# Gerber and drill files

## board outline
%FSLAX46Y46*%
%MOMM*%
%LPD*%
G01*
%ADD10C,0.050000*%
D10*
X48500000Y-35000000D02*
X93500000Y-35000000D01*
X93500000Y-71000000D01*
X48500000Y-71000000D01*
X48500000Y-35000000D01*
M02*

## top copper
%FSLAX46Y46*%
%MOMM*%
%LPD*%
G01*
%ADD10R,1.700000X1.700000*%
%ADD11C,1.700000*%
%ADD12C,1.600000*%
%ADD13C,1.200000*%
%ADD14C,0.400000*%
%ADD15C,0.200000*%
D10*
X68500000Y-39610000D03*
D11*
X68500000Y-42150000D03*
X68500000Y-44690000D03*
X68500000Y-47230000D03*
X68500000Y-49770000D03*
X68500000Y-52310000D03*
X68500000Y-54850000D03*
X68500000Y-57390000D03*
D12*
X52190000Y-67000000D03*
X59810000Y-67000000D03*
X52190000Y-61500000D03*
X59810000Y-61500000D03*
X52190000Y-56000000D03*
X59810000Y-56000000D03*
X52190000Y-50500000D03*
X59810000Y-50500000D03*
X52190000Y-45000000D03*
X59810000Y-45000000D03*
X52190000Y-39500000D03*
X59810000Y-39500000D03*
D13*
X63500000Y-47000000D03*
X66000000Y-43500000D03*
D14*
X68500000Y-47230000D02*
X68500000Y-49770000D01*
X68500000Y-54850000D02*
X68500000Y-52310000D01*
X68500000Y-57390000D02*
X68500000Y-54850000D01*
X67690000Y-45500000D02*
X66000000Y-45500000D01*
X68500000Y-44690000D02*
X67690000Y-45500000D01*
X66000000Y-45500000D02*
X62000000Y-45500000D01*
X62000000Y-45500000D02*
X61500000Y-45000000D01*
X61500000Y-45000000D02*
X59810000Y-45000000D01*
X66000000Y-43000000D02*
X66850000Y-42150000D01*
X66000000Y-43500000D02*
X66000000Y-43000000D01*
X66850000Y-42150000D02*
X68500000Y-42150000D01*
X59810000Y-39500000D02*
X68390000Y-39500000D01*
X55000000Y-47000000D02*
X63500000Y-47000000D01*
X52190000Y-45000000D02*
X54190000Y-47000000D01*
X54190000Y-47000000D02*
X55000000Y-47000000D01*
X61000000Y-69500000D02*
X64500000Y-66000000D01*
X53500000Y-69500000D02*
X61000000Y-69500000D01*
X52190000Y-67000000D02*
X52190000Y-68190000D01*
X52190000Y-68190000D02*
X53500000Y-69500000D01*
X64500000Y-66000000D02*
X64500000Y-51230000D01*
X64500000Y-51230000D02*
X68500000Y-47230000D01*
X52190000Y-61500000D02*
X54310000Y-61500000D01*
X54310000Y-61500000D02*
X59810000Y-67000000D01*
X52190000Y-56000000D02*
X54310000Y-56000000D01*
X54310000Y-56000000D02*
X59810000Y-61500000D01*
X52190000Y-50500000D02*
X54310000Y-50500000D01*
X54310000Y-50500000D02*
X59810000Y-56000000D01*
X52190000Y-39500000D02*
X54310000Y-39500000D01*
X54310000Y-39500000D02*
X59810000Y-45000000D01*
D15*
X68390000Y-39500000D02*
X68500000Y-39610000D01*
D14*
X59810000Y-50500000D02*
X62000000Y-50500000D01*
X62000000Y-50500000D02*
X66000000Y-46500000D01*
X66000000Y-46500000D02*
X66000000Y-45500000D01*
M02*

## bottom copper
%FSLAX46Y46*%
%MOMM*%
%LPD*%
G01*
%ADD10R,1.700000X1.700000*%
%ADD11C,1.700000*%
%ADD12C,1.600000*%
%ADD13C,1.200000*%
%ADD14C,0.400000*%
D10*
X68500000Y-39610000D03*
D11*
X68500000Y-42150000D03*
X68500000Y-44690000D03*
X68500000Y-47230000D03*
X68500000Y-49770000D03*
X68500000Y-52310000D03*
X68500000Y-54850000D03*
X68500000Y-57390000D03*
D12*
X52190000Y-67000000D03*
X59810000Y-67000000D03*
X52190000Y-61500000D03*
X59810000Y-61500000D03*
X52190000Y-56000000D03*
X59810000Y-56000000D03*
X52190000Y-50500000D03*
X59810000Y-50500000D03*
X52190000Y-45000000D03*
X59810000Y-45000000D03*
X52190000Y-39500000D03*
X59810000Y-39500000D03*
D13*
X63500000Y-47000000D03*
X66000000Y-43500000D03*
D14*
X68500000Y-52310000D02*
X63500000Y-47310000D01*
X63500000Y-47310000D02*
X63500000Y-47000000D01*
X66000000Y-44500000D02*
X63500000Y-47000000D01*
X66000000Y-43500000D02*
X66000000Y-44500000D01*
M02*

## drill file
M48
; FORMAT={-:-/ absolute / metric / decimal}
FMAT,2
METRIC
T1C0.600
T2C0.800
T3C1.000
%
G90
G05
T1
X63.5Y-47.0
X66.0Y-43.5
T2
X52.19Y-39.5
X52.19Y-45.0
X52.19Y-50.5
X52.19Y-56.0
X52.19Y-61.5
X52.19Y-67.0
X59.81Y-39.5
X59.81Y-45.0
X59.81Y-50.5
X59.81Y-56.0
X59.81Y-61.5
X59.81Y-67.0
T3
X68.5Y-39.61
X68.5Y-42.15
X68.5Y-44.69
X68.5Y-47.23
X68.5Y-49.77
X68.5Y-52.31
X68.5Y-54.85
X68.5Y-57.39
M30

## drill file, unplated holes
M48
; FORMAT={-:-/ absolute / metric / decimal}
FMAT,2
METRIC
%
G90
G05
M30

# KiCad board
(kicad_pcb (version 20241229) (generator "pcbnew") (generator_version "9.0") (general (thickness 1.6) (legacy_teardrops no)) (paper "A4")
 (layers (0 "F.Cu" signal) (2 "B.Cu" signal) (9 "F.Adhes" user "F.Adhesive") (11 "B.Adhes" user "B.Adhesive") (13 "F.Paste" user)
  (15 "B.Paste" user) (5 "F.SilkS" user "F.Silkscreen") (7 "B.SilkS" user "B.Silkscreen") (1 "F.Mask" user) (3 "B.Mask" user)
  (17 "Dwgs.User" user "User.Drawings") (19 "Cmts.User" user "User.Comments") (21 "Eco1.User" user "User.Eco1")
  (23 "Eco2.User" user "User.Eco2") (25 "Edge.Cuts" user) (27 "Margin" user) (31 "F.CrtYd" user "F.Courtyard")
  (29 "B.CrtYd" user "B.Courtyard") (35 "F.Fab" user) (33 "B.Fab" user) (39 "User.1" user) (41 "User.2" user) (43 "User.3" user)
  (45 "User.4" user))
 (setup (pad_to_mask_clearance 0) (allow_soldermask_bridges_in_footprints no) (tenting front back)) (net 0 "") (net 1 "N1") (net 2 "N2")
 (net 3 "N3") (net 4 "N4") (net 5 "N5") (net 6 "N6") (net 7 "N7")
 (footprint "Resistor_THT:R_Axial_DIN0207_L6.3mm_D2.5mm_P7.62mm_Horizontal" (layer "F.Cu") (at 52.19 45)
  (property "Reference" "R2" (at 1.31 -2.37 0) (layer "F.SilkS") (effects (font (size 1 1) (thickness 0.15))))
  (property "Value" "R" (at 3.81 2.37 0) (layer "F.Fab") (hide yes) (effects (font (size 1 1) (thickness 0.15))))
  (pad "1" thru_hole circle (at 0 0) (size 1.6 1.6) (drill 0.8) (layers "*.Cu" "*.Mask") (remove_unused_layers no) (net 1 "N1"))
  (pad "2" thru_hole circle (at 7.62 0) (size 1.6 1.6) (drill 0.8) (layers "*.Cu" "*.Mask") (remove_unused_layers no) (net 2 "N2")))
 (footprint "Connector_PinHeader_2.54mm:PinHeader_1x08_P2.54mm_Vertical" (layer "F.Cu") (at 68.5 39.61)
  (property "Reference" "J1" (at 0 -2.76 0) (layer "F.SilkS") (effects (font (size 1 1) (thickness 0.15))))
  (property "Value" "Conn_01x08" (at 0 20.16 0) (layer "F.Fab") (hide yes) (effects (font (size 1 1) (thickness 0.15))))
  (pad "1" thru_hole rect (at 0 0) (size 1.7 1.7) (drill 1) (layers "*.Cu" "*.Mask") (remove_unused_layers no) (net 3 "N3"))
  (pad "2" thru_hole circle (at 0 2.54) (size 1.7 1.7) (drill 1) (layers "*.Cu" "*.Mask") (remove_unused_layers no) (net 1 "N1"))
  (pad "3" thru_hole circle (at 0 5.08) (size 1.7 1.7) (drill 1) (layers "*.Cu" "*.Mask") (remove_unused_layers no) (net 2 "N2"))
  (pad "4" thru_hole circle (at 0 7.62) (size 1.7 1.7) (drill 1) (layers "*.Cu" "*.Mask") (remove_unused_layers no) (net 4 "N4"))
  (pad "5" thru_hole circle (at 0 10.16) (size 1.7 1.7) (drill 1) (layers "*.Cu" "*.Mask") (remove_unused_layers no) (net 4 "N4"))
  (pad "6" thru_hole circle (at 0 12.7) (size 1.7 1.7) (drill 1) (layers "*.Cu" "*.Mask") (remove_unused_layers no) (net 1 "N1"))
  (pad "7" thru_hole circle (at 0 15.24) (size 1.7 1.7) (drill 1) (layers "*.Cu" "*.Mask") (remove_unused_layers no) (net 1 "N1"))
  (pad "8" thru_hole circle (at 0 17.78) (size 1.7 1.7) (drill 1) (layers "*.Cu" "*.Mask") (remove_unused_layers no) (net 1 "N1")))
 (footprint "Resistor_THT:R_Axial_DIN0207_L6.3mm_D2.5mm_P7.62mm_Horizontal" (layer "F.Cu") (at 52.19 61.5)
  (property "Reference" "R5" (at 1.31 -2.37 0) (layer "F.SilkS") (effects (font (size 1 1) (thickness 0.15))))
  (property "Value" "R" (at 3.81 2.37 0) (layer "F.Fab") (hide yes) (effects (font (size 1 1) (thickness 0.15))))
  (pad "1" thru_hole circle (at 0 0) (size 1.6 1.6) (drill 0.8) (layers "*.Cu" "*.Mask") (remove_unused_layers no) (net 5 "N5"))
  (pad "2" thru_hole circle (at 7.62 0) (size 1.6 1.6) (drill 0.8) (layers "*.Cu" "*.Mask") (remove_unused_layers no) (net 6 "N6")))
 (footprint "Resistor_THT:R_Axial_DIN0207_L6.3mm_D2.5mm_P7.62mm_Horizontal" (layer "F.Cu") (at 52.19 67)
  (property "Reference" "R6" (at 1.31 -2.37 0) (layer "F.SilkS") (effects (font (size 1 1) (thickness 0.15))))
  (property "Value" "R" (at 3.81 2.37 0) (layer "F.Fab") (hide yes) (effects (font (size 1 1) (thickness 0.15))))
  (pad "1" thru_hole circle (at 0 0) (size 1.6 1.6) (drill 0.8) (layers "*.Cu" "*.Mask") (remove_unused_layers no) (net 4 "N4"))
  (pad "2" thru_hole circle (at 7.62 0) (size 1.6 1.6) (drill 0.8) (layers "*.Cu" "*.Mask") (remove_unused_layers no) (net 5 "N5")))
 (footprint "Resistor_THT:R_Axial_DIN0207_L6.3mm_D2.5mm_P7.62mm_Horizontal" (layer "F.Cu") (at 52.19 39.5)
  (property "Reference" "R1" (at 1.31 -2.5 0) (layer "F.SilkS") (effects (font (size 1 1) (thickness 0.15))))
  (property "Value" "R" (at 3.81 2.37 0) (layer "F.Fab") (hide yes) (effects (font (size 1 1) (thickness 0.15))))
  (pad "1" thru_hole circle (at 0 0) (size 1.6 1.6) (drill 0.8) (layers "*.Cu" "*.Mask") (remove_unused_layers no) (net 2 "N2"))
  (pad "2" thru_hole circle (at 7.62 0) (size 1.6 1.6) (drill 0.8) (layers "*.Cu" "*.Mask") (remove_unused_layers no) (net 3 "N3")))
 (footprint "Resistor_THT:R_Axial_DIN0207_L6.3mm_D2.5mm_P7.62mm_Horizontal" (layer "F.Cu") (at 52.19 50.5)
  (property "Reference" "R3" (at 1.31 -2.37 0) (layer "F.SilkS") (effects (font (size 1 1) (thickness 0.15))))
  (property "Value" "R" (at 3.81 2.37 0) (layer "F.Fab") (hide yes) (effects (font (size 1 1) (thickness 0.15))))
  (pad "1" thru_hole circle (at 0 0) (size 1.6 1.6) (drill 0.8) (layers "*.Cu" "*.Mask") (remove_unused_layers no) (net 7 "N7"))
  (pad "2" thru_hole circle (at 7.62 0) (size 1.6 1.6) (drill 0.8) (layers "*.Cu" "*.Mask") (remove_unused_layers no) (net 2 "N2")))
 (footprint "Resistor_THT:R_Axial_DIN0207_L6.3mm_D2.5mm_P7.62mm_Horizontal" (layer "F.Cu") (at 52.19 56)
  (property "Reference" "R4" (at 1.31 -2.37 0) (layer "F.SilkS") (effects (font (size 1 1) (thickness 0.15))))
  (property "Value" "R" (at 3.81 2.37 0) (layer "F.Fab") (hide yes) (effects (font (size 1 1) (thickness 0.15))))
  (pad "1" thru_hole circle (at 0 0) (size 1.6 1.6) (drill 0.8) (layers "*.Cu" "*.Mask") (remove_unused_layers no) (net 6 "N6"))
  (pad "2" thru_hole circle (at 7.62 0) (size 1.6 1.6) (drill 0.8) (layers "*.Cu" "*.Mask") (remove_unused_layers no) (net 7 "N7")))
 (gr_rect (start 48.5 35) (end 93.5 71) (stroke (width 0.05) (type default)) (fill no) (layer "Edge.Cuts"))
 (segment (start 61.5 45) (end 59.81 45) (width 0.4) (layer "F.Cu") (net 2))
 (segment (start 66 46.5) (end 66 45.5) (width 0.4) (layer "F.Cu") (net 2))
 (segment (start 67.69 45.5) (end 66 45.5) (width 0.4) (layer "F.Cu") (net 2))
 (segment (start 66 45.5) (end 62 45.5) (width 0.4) (layer "F.Cu") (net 2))
 (segment (start 59.81 50.5) (end 62 50.5) (width 0.4) (layer "F.Cu") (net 2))
 (segment (start 54.31 39.5) (end 59.81 45) (width 0.4) (layer "F.Cu") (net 2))
 (segment (start 62 50.5) (end 66 46.5) (width 0.4) (layer "F.Cu") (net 2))
 (segment (start 68.5 44.69) (end 67.69 45.5) (width 0.4) (layer "F.Cu") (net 2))
 (segment (start 52.19 39.5) (end 54.31 39.5) (width 0.4) (layer "F.Cu") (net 2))
 (segment (start 62 45.5) (end 61.5 45) (width 0.4) (layer "F.Cu") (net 2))
 (segment (start 59.81 39.5) (end 68.39 39.5) (width 0.4) (layer "F.Cu") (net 3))
 (segment (start 68.39 39.5) (end 68.5 39.61) (width 0.2) (layer "F.Cu") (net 3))
 (segment (start 68.5 47.23) (end 68.5 49.77) (width 0.4) (layer "F.Cu") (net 4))
 (segment (start 53.5 69.5) (end 61 69.5) (width 0.4) (layer "F.Cu") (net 4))
 (segment (start 64.5 66) (end 64.5 51.23) (width 0.4) (layer "F.Cu") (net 4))
 (segment (start 52.19 68.19) (end 53.5 69.5) (width 0.4) (layer "F.Cu") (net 4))
 (segment (start 64.5 51.23) (end 68.5 47.23) (width 0.4) (layer "F.Cu") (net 4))
 (segment (start 52.19 67) (end 52.19 68.19) (width 0.4) (layer "F.Cu") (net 4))
 (segment (start 61 69.5) (end 64.5 66) (width 0.4) (layer "F.Cu") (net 4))
 (segment (start 68.5 54.85) (end 68.5 52.31) (width 0.4) (layer "F.Cu") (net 1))
 (segment (start 66 43) (end 66.85 42.15) (width 0.4) (layer "F.Cu") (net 1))
 (segment (start 66 43.5) (end 66 43) (width 0.4) (layer "F.Cu") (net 1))
 (segment (start 55 47) (end 63.5 47) (width 0.4) (layer "F.Cu") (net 1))
 (segment (start 66.85 42.15) (end 68.5 42.15) (width 0.4) (layer "F.Cu") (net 1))
 (segment (start 68.5 57.39) (end 68.5 54.85) (width 0.4) (layer "F.Cu") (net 1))
 (segment (start 52.19 45) (end 54.19 47) (width 0.4) (layer "F.Cu") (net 1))
 (segment (start 54.19 47) (end 55 47) (width 0.4) (layer "F.Cu") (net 1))
 (via (at 66 43.5) (size 1.2) (drill 0.6) (layers "F.Cu" "B.Cu") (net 1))
 (via (at 63.5 47) (size 1.2) (drill 0.6) (layers "F.Cu" "B.Cu") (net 1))
 (segment (start 66 43.5) (end 66 44.5) (width 0.4) (layer "B.Cu") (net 1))
 (segment (start 66 44.5) (end 63.5 47) (width 0.4) (layer "B.Cu") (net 1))
 (segment (start 68.5 52.31) (end 63.5 47.31) (width 0.4) (layer "B.Cu") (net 1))
 (segment (start 63.5 47.31) (end 63.5 47) (width 0.4) (layer "B.Cu") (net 1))
 (segment (start 54.31 50.5) (end 59.81 56) (width 0.4) (layer "F.Cu") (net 7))
 (segment (start 52.19 50.5) (end 54.31 50.5) (width 0.4) (layer "F.Cu") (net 7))
 (segment (start 52.19 56) (end 54.31 56) (width 0.4) (layer "F.Cu") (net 6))
 (segment (start 54.31 56) (end 59.81 61.5) (width 0.4) (layer "F.Cu") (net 6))
 (segment (start 52.19 61.5) (end 54.31 61.5) (width 0.4) (layer "F.Cu") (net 5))
 (segment (start 54.31 61.5) (end 59.81 67) (width 0.4) (layer "F.Cu") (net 5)))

